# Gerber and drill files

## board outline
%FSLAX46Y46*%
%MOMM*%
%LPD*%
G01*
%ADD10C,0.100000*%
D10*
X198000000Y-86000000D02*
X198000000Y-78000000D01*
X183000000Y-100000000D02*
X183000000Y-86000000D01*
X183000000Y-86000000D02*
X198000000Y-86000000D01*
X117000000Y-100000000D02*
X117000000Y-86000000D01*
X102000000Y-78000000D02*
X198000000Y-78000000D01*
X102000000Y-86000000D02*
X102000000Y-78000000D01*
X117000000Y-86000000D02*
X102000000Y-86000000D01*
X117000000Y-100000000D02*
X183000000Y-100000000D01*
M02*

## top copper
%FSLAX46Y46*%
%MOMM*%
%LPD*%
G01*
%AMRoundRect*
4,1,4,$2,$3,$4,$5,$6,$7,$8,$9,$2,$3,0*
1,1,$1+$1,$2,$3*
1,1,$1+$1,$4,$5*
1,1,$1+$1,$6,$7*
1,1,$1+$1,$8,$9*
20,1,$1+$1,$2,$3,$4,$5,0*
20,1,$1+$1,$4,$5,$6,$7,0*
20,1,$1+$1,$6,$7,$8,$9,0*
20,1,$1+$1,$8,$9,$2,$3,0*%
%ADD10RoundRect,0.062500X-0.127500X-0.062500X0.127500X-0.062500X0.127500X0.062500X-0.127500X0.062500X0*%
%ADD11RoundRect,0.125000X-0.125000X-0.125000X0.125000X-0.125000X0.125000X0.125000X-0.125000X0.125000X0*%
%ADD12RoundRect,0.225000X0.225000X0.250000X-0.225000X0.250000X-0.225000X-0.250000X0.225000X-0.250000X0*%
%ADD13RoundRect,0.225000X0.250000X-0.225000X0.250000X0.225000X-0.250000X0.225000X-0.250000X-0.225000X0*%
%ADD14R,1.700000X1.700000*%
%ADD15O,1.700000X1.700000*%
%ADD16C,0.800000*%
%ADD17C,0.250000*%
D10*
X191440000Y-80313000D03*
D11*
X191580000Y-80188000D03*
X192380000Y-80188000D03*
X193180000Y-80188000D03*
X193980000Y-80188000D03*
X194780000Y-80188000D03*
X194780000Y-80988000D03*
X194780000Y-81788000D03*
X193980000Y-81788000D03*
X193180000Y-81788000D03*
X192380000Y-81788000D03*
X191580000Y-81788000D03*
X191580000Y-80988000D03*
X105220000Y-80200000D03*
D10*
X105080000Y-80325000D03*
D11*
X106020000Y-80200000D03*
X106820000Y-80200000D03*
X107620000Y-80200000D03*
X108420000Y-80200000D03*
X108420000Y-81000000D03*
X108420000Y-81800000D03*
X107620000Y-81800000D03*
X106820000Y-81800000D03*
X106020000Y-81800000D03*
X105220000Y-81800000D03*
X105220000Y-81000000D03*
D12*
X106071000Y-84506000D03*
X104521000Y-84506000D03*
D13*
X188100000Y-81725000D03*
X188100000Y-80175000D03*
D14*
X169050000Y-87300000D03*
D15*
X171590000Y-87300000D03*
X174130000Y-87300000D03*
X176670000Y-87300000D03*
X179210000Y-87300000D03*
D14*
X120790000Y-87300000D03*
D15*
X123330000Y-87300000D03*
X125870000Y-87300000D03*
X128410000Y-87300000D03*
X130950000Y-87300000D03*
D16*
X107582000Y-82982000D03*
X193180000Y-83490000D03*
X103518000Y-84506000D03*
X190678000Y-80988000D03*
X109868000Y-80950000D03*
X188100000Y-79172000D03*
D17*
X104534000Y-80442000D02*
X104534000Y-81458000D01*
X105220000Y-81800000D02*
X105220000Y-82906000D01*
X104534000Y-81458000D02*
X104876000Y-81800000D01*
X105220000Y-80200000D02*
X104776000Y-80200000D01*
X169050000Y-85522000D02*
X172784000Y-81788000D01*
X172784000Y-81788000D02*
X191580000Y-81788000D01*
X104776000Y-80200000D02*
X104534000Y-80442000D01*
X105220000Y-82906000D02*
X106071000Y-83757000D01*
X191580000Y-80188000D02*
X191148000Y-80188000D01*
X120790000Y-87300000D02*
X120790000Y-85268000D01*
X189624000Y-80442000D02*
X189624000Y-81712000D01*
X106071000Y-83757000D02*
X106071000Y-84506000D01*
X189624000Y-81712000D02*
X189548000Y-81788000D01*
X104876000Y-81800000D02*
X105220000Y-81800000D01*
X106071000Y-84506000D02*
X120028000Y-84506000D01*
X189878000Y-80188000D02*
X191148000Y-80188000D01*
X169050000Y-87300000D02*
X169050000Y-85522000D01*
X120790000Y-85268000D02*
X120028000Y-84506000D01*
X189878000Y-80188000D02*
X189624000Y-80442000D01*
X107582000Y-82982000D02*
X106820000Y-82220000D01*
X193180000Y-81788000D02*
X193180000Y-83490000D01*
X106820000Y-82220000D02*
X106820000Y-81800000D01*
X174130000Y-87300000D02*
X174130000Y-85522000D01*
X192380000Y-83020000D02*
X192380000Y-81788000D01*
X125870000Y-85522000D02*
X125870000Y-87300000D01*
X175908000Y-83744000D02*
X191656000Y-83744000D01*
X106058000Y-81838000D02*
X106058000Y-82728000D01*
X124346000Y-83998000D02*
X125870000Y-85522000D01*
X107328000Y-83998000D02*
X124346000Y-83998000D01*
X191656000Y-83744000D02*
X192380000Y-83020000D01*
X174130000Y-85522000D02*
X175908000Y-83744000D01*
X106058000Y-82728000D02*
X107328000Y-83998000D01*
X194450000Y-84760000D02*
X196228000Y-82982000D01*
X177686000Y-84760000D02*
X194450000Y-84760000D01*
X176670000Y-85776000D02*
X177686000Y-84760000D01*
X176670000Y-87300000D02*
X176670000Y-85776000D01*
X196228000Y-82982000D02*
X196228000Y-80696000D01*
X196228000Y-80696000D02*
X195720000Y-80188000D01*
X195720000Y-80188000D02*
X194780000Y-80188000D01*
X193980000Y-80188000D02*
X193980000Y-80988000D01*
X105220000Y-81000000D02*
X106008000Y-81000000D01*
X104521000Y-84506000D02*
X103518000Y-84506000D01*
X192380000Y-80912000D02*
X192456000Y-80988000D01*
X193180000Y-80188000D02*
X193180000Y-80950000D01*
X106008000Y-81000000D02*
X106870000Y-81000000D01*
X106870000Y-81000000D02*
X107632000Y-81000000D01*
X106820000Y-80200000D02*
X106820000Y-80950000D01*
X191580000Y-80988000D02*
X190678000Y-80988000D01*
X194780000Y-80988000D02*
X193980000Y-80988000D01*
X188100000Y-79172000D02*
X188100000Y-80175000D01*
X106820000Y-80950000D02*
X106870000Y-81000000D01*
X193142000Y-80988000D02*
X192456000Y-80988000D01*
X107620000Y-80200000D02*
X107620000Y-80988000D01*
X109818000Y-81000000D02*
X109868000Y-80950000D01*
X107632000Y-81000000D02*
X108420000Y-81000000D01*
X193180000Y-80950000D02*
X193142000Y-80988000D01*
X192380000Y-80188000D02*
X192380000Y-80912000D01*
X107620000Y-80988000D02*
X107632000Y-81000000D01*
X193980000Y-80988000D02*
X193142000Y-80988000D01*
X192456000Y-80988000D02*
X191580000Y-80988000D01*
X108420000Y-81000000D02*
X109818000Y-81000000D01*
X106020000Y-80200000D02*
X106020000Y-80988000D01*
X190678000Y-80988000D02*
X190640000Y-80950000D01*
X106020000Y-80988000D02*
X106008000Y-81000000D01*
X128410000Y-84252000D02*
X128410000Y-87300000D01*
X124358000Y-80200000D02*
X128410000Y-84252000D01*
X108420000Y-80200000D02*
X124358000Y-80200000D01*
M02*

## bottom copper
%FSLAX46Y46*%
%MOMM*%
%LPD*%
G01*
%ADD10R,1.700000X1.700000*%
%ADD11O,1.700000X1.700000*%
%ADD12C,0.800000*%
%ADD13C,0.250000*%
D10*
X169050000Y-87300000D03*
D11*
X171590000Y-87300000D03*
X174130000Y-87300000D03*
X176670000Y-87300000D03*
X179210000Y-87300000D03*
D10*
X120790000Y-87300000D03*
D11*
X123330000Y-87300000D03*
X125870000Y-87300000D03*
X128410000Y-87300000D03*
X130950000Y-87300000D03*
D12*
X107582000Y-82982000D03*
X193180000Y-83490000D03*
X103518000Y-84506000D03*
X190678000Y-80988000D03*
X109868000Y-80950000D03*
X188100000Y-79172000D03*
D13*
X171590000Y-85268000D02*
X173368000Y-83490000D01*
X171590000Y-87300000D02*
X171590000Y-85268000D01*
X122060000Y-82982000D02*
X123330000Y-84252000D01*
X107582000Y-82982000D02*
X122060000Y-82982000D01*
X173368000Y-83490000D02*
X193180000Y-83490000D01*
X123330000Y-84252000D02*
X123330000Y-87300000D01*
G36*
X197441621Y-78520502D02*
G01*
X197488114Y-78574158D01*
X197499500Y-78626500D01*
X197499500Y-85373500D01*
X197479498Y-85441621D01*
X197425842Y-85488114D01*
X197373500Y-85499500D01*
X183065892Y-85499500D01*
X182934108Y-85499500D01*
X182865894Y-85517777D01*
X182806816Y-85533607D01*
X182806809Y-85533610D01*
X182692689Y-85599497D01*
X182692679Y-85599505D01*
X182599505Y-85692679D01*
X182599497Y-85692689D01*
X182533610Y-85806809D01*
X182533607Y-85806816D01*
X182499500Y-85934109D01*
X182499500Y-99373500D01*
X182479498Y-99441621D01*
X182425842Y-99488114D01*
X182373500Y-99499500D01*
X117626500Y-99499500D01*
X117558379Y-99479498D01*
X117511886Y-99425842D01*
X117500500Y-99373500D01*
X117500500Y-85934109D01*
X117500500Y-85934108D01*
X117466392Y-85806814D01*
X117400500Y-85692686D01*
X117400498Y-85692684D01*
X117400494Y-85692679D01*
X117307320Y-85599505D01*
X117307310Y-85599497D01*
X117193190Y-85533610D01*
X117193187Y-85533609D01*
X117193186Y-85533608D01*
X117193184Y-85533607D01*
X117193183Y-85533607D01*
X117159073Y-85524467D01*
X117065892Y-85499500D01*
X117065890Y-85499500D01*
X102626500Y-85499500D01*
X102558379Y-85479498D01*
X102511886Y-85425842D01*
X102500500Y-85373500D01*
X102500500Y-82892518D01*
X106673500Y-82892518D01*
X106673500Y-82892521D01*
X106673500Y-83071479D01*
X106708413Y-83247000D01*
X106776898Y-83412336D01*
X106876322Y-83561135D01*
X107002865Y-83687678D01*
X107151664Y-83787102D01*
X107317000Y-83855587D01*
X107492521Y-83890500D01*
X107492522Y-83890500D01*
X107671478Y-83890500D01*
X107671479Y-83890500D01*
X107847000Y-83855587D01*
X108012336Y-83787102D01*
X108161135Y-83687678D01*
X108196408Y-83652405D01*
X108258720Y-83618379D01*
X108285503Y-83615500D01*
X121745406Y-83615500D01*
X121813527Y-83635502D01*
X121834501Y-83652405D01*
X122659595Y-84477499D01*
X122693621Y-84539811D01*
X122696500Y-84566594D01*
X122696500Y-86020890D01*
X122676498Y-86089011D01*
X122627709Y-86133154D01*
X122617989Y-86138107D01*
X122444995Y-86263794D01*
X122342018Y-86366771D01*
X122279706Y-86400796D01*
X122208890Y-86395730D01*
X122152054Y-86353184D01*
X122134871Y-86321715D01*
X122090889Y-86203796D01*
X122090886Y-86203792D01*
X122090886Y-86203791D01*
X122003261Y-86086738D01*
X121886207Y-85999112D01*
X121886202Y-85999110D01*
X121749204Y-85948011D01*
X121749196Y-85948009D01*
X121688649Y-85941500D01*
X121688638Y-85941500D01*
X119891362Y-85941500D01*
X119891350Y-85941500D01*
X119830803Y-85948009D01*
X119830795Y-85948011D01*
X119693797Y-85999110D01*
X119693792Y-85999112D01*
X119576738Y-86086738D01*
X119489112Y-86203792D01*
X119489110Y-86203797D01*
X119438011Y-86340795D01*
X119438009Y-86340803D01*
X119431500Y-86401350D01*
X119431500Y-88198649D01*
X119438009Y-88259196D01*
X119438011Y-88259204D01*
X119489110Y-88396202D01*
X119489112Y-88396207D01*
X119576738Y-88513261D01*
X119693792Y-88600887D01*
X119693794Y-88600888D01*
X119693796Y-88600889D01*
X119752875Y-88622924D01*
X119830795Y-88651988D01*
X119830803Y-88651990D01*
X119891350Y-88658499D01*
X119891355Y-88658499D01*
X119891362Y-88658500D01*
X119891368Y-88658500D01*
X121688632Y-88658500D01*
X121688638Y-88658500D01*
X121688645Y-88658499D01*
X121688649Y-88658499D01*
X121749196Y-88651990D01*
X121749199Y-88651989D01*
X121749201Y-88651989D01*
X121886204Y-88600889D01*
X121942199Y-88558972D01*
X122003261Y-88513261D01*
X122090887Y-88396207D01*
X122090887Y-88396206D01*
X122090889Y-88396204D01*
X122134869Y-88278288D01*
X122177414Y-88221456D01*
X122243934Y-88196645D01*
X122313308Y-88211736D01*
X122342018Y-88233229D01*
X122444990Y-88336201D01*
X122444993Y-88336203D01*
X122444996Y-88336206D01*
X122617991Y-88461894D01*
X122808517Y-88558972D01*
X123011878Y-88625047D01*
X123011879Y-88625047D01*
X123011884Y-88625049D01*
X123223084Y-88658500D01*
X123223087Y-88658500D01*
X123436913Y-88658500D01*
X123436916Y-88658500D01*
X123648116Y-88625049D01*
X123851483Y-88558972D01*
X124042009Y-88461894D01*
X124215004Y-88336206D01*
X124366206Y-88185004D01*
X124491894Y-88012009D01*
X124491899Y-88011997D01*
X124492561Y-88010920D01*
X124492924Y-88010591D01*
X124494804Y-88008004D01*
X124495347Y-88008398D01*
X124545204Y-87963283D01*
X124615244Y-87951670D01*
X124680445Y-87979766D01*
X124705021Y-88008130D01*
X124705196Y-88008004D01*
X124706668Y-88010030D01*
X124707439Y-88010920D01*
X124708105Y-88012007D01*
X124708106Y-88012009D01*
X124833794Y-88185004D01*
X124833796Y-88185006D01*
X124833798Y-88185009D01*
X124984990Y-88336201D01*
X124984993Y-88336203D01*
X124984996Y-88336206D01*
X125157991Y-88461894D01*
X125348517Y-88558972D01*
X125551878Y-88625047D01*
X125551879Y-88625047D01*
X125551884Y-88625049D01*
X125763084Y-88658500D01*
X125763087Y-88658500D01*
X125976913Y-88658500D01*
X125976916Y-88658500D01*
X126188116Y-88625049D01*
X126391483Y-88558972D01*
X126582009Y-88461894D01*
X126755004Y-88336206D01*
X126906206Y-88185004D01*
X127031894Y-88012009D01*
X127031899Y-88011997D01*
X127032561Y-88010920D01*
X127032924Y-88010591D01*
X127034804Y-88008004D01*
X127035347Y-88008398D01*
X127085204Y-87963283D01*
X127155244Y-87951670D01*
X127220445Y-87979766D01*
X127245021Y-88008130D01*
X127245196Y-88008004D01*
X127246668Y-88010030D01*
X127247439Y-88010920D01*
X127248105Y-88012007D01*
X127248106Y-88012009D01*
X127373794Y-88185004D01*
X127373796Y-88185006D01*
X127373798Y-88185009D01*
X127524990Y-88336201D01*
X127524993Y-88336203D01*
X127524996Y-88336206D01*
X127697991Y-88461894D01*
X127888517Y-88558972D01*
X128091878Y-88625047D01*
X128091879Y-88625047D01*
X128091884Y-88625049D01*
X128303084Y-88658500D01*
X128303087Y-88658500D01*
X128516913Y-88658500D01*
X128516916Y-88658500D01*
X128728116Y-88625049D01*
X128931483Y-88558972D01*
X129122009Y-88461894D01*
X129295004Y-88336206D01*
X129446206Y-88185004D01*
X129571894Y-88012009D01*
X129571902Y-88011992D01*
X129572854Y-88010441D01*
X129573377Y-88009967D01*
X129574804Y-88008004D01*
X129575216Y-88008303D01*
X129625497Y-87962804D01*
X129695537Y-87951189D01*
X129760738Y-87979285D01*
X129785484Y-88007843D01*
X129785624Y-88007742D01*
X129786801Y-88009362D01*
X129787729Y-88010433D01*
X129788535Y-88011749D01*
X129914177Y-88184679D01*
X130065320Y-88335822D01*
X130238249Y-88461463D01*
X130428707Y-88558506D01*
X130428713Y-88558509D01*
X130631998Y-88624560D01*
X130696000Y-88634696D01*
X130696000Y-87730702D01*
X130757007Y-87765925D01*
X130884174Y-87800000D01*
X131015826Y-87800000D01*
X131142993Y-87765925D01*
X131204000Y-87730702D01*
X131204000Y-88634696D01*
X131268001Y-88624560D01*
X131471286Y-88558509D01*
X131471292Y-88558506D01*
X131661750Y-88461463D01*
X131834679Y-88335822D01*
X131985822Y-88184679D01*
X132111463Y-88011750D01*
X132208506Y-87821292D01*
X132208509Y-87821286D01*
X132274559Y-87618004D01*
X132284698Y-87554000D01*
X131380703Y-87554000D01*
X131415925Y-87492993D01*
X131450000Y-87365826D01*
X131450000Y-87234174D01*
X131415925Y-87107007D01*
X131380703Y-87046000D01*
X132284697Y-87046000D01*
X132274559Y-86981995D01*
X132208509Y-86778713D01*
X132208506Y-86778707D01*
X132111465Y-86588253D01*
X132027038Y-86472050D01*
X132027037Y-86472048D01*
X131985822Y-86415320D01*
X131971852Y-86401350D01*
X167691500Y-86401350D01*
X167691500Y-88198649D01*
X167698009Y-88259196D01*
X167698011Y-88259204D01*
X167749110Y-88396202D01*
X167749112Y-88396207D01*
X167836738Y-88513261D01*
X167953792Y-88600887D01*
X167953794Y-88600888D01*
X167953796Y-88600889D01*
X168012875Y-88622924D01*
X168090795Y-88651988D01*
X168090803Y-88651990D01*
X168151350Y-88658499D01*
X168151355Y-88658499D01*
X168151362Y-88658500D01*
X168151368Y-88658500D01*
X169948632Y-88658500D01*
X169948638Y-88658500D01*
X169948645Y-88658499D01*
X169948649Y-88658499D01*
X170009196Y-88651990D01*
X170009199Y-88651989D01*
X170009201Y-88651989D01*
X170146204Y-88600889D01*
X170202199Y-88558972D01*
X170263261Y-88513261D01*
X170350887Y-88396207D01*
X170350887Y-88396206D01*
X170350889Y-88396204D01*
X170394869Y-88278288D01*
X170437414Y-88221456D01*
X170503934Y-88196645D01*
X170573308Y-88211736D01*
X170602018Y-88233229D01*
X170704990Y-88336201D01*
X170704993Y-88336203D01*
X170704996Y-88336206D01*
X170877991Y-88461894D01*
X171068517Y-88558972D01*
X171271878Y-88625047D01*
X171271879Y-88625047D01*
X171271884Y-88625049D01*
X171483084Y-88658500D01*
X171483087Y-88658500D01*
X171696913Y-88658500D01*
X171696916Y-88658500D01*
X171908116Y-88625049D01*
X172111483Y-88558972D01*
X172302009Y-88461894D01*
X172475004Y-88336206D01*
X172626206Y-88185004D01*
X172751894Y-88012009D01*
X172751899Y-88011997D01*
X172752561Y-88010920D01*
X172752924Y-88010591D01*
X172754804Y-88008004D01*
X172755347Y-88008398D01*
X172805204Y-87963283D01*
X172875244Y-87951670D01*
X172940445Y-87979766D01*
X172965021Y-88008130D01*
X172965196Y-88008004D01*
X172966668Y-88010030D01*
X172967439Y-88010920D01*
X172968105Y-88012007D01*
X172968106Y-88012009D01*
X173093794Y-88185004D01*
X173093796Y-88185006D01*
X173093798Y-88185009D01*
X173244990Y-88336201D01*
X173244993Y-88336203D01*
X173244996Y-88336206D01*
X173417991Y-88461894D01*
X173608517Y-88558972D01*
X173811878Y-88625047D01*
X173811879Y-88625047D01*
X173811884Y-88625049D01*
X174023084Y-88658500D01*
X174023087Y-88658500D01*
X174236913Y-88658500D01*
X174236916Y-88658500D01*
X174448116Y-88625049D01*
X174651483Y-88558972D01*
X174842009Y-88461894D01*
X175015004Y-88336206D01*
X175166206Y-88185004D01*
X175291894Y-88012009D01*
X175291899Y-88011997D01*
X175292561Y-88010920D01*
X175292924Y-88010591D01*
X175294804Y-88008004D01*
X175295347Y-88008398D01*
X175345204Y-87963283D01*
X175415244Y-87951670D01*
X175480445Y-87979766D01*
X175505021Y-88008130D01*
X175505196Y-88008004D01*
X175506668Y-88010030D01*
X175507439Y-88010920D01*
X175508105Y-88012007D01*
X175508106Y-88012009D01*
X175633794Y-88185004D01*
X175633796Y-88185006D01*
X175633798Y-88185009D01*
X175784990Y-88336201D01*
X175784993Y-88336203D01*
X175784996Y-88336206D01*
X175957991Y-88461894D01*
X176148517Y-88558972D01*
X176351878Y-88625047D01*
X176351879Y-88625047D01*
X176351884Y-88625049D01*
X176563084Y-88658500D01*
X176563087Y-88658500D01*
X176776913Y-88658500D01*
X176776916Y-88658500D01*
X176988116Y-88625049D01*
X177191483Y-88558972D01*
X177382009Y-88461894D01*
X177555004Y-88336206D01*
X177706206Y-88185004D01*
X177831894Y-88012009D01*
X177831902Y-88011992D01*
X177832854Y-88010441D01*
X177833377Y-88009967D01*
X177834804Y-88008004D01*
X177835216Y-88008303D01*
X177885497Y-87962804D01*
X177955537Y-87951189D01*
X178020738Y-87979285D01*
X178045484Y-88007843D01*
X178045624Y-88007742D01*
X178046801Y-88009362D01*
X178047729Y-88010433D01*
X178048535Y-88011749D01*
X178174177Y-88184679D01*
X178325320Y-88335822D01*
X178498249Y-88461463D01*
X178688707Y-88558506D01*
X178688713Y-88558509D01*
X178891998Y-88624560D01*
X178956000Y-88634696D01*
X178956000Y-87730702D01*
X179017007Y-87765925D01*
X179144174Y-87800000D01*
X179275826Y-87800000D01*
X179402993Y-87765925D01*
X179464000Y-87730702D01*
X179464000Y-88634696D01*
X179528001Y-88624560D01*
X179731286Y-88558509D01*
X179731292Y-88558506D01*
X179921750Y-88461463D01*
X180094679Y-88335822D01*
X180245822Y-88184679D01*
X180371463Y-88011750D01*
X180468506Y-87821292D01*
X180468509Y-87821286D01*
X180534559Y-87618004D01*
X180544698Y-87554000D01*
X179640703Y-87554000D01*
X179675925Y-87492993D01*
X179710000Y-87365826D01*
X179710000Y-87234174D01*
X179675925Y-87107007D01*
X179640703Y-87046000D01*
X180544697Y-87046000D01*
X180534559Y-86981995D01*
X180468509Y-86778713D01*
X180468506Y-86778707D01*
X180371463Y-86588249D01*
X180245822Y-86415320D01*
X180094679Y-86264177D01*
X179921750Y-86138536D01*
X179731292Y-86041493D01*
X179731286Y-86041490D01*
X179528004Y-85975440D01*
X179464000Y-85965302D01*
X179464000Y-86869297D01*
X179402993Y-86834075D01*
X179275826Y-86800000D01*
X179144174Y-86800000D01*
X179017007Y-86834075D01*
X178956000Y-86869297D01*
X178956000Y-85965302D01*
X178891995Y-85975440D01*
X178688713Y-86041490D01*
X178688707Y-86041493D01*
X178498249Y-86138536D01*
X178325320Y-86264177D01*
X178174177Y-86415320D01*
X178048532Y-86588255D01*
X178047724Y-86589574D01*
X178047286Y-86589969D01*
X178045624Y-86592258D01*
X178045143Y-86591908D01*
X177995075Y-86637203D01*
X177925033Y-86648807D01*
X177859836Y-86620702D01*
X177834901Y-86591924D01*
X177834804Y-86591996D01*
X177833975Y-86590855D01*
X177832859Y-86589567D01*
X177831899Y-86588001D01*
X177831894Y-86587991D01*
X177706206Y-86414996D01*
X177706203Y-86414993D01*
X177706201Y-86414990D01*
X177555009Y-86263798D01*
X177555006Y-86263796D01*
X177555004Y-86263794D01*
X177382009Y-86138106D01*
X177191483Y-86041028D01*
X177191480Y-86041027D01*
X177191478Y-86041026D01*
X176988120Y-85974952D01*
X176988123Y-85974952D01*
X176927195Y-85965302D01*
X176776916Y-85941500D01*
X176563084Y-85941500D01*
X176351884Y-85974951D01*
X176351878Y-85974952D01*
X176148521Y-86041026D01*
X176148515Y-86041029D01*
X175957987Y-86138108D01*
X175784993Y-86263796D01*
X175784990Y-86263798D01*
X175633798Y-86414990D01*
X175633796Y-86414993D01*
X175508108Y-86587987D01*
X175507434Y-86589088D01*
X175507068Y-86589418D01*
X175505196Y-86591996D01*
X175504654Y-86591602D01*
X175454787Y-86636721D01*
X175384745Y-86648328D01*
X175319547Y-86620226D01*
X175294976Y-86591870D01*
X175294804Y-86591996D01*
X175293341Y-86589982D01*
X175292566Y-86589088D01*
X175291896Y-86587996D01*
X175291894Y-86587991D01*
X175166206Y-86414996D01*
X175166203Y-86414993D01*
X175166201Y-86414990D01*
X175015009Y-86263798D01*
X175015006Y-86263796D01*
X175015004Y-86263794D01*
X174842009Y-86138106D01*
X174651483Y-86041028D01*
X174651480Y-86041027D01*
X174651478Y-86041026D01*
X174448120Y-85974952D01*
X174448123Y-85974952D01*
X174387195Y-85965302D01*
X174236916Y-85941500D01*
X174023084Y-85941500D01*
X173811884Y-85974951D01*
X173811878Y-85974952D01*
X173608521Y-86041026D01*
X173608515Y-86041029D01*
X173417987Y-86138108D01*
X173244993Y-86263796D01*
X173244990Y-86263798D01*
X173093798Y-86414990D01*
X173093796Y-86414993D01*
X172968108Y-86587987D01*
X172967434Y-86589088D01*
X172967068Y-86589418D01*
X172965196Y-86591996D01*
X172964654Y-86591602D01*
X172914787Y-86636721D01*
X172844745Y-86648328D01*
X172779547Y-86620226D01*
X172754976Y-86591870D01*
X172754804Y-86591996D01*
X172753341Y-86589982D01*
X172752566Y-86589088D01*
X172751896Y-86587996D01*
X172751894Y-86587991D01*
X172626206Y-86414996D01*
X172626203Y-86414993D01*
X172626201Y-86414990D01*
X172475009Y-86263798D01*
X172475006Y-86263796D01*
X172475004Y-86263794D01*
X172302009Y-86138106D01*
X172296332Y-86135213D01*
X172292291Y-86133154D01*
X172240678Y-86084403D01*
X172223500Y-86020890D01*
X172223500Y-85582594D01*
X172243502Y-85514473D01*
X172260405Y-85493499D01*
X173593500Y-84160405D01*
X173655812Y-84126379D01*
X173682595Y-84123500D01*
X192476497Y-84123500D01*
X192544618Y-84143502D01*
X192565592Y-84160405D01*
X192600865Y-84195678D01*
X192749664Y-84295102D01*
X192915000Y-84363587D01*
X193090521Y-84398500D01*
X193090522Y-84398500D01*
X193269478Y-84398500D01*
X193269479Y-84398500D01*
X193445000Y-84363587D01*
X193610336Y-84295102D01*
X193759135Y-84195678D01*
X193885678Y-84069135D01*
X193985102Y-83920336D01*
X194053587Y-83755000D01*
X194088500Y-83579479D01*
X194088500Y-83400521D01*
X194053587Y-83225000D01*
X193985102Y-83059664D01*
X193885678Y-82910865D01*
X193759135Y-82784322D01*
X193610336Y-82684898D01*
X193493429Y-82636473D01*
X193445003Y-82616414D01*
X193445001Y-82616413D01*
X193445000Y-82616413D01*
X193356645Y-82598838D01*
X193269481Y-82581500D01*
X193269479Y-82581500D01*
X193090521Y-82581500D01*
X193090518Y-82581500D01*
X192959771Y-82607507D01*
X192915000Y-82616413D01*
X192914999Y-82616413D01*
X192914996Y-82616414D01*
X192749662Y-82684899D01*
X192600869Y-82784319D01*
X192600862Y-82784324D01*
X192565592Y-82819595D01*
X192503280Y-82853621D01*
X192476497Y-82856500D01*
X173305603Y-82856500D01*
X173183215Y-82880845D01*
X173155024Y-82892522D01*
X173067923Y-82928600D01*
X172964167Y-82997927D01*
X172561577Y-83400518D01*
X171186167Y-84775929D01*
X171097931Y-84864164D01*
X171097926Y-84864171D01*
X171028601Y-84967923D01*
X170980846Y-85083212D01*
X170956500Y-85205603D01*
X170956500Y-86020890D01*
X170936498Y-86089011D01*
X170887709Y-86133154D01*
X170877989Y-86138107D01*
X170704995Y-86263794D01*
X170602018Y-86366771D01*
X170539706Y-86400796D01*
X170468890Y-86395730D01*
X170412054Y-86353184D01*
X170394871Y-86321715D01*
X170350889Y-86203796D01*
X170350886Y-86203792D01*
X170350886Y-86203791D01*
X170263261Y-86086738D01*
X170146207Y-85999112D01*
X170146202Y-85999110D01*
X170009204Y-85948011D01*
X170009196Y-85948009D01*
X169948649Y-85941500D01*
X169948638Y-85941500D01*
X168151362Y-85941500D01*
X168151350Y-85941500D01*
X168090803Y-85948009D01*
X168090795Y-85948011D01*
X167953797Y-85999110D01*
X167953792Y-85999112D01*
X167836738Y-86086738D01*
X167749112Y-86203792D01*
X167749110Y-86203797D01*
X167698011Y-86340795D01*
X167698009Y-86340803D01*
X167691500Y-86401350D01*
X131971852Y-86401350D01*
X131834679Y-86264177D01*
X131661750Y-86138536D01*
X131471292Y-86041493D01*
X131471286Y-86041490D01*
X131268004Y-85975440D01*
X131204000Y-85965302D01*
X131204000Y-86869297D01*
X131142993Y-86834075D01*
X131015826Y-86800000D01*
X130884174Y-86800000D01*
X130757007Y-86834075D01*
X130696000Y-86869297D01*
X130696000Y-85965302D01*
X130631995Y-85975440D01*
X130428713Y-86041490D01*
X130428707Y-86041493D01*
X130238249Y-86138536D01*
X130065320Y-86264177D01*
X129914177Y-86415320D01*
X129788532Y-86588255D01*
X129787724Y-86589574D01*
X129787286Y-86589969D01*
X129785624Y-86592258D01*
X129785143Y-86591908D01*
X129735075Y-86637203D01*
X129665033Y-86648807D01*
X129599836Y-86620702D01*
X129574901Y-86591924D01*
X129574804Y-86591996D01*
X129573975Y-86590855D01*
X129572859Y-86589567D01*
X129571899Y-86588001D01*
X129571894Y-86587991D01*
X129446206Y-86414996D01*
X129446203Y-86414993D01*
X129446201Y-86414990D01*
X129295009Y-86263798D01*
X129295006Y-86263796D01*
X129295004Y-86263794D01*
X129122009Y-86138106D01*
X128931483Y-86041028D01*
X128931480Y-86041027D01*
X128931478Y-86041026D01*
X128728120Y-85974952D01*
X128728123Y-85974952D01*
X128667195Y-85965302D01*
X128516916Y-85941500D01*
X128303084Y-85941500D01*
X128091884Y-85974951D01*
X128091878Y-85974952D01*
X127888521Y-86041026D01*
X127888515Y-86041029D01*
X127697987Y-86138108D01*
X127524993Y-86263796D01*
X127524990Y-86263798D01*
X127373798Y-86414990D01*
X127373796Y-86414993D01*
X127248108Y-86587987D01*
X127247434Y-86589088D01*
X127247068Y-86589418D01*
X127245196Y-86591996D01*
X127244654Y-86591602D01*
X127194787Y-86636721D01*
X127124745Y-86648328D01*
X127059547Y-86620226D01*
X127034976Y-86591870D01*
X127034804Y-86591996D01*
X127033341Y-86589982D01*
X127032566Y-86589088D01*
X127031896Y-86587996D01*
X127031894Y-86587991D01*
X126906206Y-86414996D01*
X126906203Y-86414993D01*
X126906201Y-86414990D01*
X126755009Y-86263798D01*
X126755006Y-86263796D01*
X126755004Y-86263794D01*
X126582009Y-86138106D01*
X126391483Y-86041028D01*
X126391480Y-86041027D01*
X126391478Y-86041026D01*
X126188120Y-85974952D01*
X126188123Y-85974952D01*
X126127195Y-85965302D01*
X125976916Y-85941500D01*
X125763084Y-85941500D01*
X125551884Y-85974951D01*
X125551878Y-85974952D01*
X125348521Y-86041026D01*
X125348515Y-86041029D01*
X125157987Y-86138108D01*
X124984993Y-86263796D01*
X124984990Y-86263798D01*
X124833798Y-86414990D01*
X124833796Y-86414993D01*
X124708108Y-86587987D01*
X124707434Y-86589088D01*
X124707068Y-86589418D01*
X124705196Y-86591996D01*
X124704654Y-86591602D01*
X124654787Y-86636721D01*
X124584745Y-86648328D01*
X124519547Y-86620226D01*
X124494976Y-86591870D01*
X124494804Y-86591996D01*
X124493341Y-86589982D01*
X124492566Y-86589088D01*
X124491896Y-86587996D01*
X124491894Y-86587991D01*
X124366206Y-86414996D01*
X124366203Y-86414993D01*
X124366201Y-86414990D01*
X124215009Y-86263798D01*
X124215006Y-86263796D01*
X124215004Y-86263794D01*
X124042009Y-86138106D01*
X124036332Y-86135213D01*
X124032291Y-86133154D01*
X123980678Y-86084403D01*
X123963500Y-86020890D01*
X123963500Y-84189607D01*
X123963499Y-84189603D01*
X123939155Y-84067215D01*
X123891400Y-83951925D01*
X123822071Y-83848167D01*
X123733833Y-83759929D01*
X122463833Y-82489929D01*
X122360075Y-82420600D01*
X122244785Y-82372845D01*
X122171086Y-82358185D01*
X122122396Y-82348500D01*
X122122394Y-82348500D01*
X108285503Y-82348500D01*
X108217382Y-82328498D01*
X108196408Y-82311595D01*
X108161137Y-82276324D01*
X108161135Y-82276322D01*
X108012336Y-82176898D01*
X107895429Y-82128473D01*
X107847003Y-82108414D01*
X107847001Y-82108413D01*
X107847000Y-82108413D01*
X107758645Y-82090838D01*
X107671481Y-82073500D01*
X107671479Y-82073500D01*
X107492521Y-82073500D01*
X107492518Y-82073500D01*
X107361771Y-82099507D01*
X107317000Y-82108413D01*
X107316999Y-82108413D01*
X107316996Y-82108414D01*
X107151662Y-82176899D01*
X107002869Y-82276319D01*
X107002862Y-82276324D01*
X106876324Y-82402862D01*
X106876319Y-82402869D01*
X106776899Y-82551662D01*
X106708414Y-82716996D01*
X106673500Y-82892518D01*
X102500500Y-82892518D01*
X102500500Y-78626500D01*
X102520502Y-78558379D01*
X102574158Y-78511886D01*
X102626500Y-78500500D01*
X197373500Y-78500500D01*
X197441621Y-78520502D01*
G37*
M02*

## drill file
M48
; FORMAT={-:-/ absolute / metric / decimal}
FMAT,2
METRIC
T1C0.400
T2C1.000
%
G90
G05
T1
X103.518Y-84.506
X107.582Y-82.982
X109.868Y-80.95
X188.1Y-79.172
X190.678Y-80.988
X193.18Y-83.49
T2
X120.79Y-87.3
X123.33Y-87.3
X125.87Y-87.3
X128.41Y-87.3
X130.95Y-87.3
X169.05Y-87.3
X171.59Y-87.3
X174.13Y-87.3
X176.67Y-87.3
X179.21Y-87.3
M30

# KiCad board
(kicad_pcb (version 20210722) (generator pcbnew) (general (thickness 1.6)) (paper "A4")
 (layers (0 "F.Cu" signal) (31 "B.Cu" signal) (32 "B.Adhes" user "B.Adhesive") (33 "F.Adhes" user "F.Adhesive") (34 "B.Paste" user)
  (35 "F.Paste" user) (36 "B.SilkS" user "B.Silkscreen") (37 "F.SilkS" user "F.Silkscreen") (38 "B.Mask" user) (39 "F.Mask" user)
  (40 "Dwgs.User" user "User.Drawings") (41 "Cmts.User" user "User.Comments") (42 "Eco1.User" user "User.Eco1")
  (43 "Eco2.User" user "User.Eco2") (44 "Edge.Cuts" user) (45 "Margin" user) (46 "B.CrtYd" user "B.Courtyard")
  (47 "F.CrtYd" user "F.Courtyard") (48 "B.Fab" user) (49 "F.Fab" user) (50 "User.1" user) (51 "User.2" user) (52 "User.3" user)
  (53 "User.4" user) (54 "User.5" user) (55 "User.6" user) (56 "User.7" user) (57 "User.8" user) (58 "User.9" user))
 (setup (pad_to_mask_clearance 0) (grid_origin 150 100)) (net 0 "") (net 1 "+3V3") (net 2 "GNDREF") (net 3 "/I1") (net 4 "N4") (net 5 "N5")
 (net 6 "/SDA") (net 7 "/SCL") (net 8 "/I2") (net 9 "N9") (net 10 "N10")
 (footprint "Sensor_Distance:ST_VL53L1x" (layer "F.Cu") (at 193.18 80.988)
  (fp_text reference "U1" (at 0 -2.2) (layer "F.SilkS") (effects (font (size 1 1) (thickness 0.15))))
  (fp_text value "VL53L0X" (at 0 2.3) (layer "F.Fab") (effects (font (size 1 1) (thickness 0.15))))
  (pad "1" smd roundrect locked (at -1.74 -0.675) (size 0.38 0.25) (layers "F.Cu" "F.Paste" "F.Mask") (roundrect_rratio 0.25) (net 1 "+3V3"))
  (pad "1" smd roundrect locked (at -1.6 -0.8) (size 0.5 0.5) (layers "F.Cu" "F.Paste" "F.Mask") (roundrect_rratio 0.25) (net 1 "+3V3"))
  (pad "2" smd roundrect locked (at -0.8 -0.8) (size 0.5 0.5) (layers "F.Cu" "F.Paste" "F.Mask") (roundrect_rratio 0.25) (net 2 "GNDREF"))
  (pad "3" smd roundrect locked (at 0 -0.8) (size 0.5 0.5) (layers "F.Cu" "F.Paste" "F.Mask") (roundrect_rratio 0.25) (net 2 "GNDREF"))
  (pad "4" smd roundrect locked (at 0.8 -0.8) (size 0.5 0.5) (layers "F.Cu" "F.Paste" "F.Mask") (roundrect_rratio 0.25) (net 2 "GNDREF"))
  (pad "5" smd roundrect locked (at 1.6 -0.8) (size 0.5 0.5) (layers "F.Cu" "F.Paste" "F.Mask") (roundrect_rratio 0.25) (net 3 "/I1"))
  (pad "6" smd roundrect locked (at 1.6 0) (size 0.5 0.5) (layers "F.Cu" "F.Paste" "F.Mask") (roundrect_rratio 0.25) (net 2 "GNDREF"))
  (pad "7" smd roundrect locked (at 1.6 0.8) (size 0.5 0.5) (layers "F.Cu" "F.Paste" "F.Mask") (roundrect_rratio 0.25) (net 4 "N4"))
  (pad "8" smd roundrect locked (at 0.8 0.8) (size 0.5 0.5) (layers "F.Cu" "F.Paste" "F.Mask") (roundrect_rratio 0.25) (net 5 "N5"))
  (pad "9" smd roundrect locked (at 0 0.8) (size 0.5 0.5) (layers "F.Cu" "F.Paste" "F.Mask") (roundrect_rratio 0.25) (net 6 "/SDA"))
  (pad "10" smd roundrect locked (at -0.8 0.8) (size 0.5 0.5) (layers "F.Cu" "F.Paste" "F.Mask") (roundrect_rratio 0.25) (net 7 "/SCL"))
  (pad "11" smd roundrect locked (at -1.6 0.8) (size 0.5 0.5) (layers "F.Cu" "F.Paste" "F.Mask") (roundrect_rratio 0.25) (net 1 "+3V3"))
  (pad "12" smd roundrect locked (at -1.6 0) (size 0.5 0.5) (layers "F.Cu" "F.Paste" "F.Mask") (roundrect_rratio 0.25) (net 2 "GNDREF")))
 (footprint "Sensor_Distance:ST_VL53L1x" (layer "F.Cu") (at 106.82 81)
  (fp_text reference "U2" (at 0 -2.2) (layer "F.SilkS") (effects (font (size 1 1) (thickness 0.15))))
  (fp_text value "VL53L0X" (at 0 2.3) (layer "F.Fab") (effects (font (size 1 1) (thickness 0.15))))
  (pad "1" smd roundrect locked (at -1.6 -0.8) (size 0.5 0.5) (layers "F.Cu" "F.Paste" "F.Mask") (roundrect_rratio 0.25) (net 1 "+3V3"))
  (pad "1" smd roundrect locked (at -1.74 -0.675) (size 0.38 0.25) (layers "F.Cu" "F.Paste" "F.Mask") (roundrect_rratio 0.25) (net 1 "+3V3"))
  (pad "2" smd roundrect locked (at -0.8 -0.8) (size 0.5 0.5) (layers "F.Cu" "F.Paste" "F.Mask") (roundrect_rratio 0.25) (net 2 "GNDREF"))
  (pad "3" smd roundrect locked (at 0 -0.8) (size 0.5 0.5) (layers "F.Cu" "F.Paste" "F.Mask") (roundrect_rratio 0.25) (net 2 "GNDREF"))
  (pad "4" smd roundrect locked (at 0.8 -0.8) (size 0.5 0.5) (layers "F.Cu" "F.Paste" "F.Mask") (roundrect_rratio 0.25) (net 2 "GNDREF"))
  (pad "5" smd roundrect locked (at 1.6 -0.8) (size 0.5 0.5) (layers "F.Cu" "F.Paste" "F.Mask") (roundrect_rratio 0.25) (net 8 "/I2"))
  (pad "6" smd roundrect locked (at 1.6 0) (size 0.5 0.5) (layers "F.Cu" "F.Paste" "F.Mask") (roundrect_rratio 0.25) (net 2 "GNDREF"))
  (pad "7" smd roundrect locked (at 1.6 0.8) (size 0.5 0.5) (layers "F.Cu" "F.Paste" "F.Mask") (roundrect_rratio 0.25) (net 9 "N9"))
  (pad "8" smd roundrect locked (at 0.8 0.8) (size 0.5 0.5) (layers "F.Cu" "F.Paste" "F.Mask") (roundrect_rratio 0.25) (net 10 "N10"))
  (pad "9" smd roundrect locked (at 0 0.8) (size 0.5 0.5) (layers "F.Cu" "F.Paste" "F.Mask") (roundrect_rratio 0.25) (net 6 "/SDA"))
  (pad "10" smd roundrect locked (at -0.8 0.8) (size 0.5 0.5) (layers "F.Cu" "F.Paste" "F.Mask") (roundrect_rratio 0.25) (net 7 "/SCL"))
  (pad "11" smd roundrect locked (at -1.6 0.8) (size 0.5 0.5) (layers "F.Cu" "F.Paste" "F.Mask") (roundrect_rratio 0.25) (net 1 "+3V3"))
  (pad "12" smd roundrect locked (at -1.6 0) (size 0.5 0.5) (layers "F.Cu" "F.Paste" "F.Mask") (roundrect_rratio 0.25) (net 2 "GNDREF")))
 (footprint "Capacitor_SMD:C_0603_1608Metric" (layer "F.Cu") (at 105.296 84.506 180)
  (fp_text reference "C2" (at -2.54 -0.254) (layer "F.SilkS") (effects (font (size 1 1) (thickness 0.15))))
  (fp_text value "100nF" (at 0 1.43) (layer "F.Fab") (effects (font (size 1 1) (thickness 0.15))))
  (pad "1" smd roundrect locked (at -0.775 0 180) (size 0.9 0.95) (layers "F.Cu" "F.Paste" "F.Mask") (roundrect_rratio 0.25) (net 1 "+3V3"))
  (pad "2" smd roundrect locked (at 0.775 0 180) (size 0.9 0.95) (layers "F.Cu" "F.Paste" "F.Mask") (roundrect_rratio 0.25) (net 2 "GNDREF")))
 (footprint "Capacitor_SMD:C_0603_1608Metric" (layer "F.Cu") (at 188.1 80.95 90)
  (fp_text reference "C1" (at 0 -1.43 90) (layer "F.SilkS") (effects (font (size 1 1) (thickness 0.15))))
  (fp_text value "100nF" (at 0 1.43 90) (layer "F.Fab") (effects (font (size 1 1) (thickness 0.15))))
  (pad "1" smd roundrect locked (at -0.775 0 90) (size 0.9 0.95) (layers "F.Cu" "F.Paste" "F.Mask") (roundrect_rratio 0.25) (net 1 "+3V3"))
  (pad "2" smd roundrect locked (at 0.775 0 90) (size 0.9 0.95) (layers "F.Cu" "F.Paste" "F.Mask") (roundrect_rratio 0.25) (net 2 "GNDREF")))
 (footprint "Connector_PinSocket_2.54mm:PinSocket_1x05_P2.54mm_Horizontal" (layer "F.Cu") (at 169.05 87.3 90)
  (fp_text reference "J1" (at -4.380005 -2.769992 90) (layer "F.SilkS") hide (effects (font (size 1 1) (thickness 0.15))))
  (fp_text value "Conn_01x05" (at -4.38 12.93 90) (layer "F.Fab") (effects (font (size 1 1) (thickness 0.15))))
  (pad "1" thru_hole rect locked (at 0 0 90) (size 1.7 1.7) (drill 1) (layers *.Cu *.Mask) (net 1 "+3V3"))
  (pad "2" thru_hole oval locked (at 0 2.54 90) (size 1.7 1.7) (drill 1) (layers *.Cu *.Mask) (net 6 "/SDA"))
  (pad "3" thru_hole oval locked (at 0 5.08 90) (size 1.7 1.7) (drill 1) (layers *.Cu *.Mask) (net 7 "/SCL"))
  (pad "4" thru_hole oval locked (at 0 7.62 90) (size 1.7 1.7) (drill 1) (layers *.Cu *.Mask) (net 3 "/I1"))
  (pad "5" thru_hole oval locked (at 0 10.16 90) (size 1.7 1.7) (drill 1) (layers *.Cu *.Mask) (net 2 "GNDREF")))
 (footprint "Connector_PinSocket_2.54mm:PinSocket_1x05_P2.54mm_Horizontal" (layer "F.Cu") (at 120.79 87.3 90)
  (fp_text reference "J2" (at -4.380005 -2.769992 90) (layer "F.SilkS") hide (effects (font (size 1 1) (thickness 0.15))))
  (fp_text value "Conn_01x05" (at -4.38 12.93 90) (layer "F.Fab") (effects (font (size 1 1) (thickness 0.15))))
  (pad "1" thru_hole rect locked (at 0 0 90) (size 1.7 1.7) (drill 1) (layers *.Cu *.Mask) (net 1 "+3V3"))
  (pad "2" thru_hole oval locked (at 0 2.54 90) (size 1.7 1.7) (drill 1) (layers *.Cu *.Mask) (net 6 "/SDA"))
  (pad "3" thru_hole oval locked (at 0 5.08 90) (size 1.7 1.7) (drill 1) (layers *.Cu *.Mask) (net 7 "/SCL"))
  (pad "4" thru_hole oval locked (at 0 7.62 90) (size 1.7 1.7) (drill 1) (layers *.Cu *.Mask) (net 8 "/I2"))
  (pad "5" thru_hole oval locked (at 0 10.16 90) (size 1.7 1.7) (drill 1) (layers *.Cu *.Mask) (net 2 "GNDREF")))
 (gr_line (start 198 86) (end 198 78) (layer "Edge.Cuts") (width 0.1))
 (gr_line (start 183 100) (end 183 86) (layer "Edge.Cuts") (width 0.1))
 (gr_line (start 183 86) (end 198 86) (layer "Edge.Cuts") (width 0.1))
 (gr_line (start 117 100) (end 117 86) (layer "Edge.Cuts") (width 0.1))
 (gr_line (start 102 78) (end 198 78) (layer "Edge.Cuts") (width 0.1))
 (gr_line (start 102 86) (end 102 78) (layer "Edge.Cuts") (width 0.1))
 (gr_line (start 117 86) (end 102 86) (layer "Edge.Cuts") (width 0.1))
 (gr_line (start 117 100) (end 183 100) (layer "Edge.Cuts") (width 0.1))
 (segment (start 104.534 80.442) (end 104.534 81.458) (width 0.25) (layer "F.Cu") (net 1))
 (segment (start 105.22 81.8) (end 105.22 82.906) (width 0.25) (layer "F.Cu") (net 1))
 (segment (start 104.534 81.458) (end 104.876 81.8) (width 0.25) (layer "F.Cu") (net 1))
 (segment (start 105.22 80.2) (end 104.776 80.2) (width 0.25) (layer "F.Cu") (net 1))
 (segment (start 169.05 85.522) (end 172.784 81.788) (width 0.25) (layer "F.Cu") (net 1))
 (segment (start 172.784 81.788) (end 191.58 81.788) (width 0.25) (layer "F.Cu") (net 1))
 (segment (start 104.776 80.2) (end 104.534 80.442) (width 0.25) (layer "F.Cu") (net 1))
 (segment (start 105.22 82.906) (end 106.071 83.757) (width 0.25) (layer "F.Cu") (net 1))
 (segment (start 191.58 80.188) (end 191.148 80.188) (width 0.25) (layer "F.Cu") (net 1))
 (segment (start 120.79 87.3) (end 120.79 85.268) (width 0.25) (layer "F.Cu") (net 1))
 (segment (start 189.624 80.442) (end 189.624 81.712) (width 0.25) (layer "F.Cu") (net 1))
 (segment (start 106.071 83.757) (end 106.071 84.506) (width 0.25) (layer "F.Cu") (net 1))
 (segment (start 189.624 81.712) (end 189.548 81.788) (width 0.25) (layer "F.Cu") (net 1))
 (segment (start 104.876 81.8) (end 105.22 81.8) (width 0.25) (layer "F.Cu") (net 1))
 (segment (start 106.071 84.506) (end 120.028 84.506) (width 0.25) (layer "F.Cu") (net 1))
 (segment (start 189.878 80.188) (end 191.148 80.188) (width 0.25) (layer "F.Cu") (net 1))
 (segment (start 169.05 87.3) (end 169.05 85.522) (width 0.25) (layer "F.Cu") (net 1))
 (segment (start 120.79 85.268) (end 120.028 84.506) (width 0.25) (layer "F.Cu") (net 1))
 (segment (start 189.878 80.188) (end 189.624 80.442) (width 0.25) (layer "F.Cu") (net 1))
 (segment (start 107.582 82.982) (end 106.82 82.22) (width 0.25) (layer "F.Cu") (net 6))
 (segment (start 193.18 81.788) (end 193.18 83.49) (width 0.25) (layer "F.Cu") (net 6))
 (segment (start 106.82 82.22) (end 106.82 81.8) (width 0.25) (layer "F.Cu") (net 6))
 (via (at 107.582 82.982) (size 0.8) (drill 0.4) (layers "F.Cu" "B.Cu") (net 6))
 (via (at 193.18 83.49) (size 0.8) (drill 0.4) (layers "F.Cu" "B.Cu") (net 6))
 (segment (start 171.59 85.268) (end 173.368 83.49) (width 0.25) (layer "B.Cu") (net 6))
 (segment (start 171.59 87.3) (end 171.59 85.268) (width 0.25) (layer "B.Cu") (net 6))
 (segment (start 122.06 82.982) (end 123.33 84.252) (width 0.25) (layer "B.Cu") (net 6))
 (segment (start 107.582 82.982) (end 122.06 82.982) (width 0.25) (layer "B.Cu") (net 6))
 (segment (start 173.368 83.49) (end 193.18 83.49) (width 0.25) (layer "B.Cu") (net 6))
 (segment (start 123.33 84.252) (end 123.33 87.3) (width 0.25) (layer "B.Cu") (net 6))
 (segment (start 174.13 87.3) (end 174.13 85.522) (width 0.25) (layer "F.Cu") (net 7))
 (segment (start 192.38 83.02) (end 192.38 81.788) (width 0.25) (layer "F.Cu") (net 7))
 (segment (start 125.87 85.522) (end 125.87 87.3) (width 0.25) (layer "F.Cu") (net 7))
 (segment (start 175.908 83.744) (end 191.656 83.744) (width 0.25) (layer "F.Cu") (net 7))
 (segment (start 106.058 81.838) (end 106.058 82.728) (width 0.25) (layer "F.Cu") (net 7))
 (segment (start 124.346 83.998) (end 125.87 85.522) (width 0.25) (layer "F.Cu") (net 7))
 (segment (start 107.328 83.998) (end 124.346 83.998) (width 0.25) (layer "F.Cu") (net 7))
 (segment (start 191.656 83.744) (end 192.38 83.02) (width 0.25) (layer "F.Cu") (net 7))
 (segment (start 174.13 85.522) (end 175.908 83.744) (width 0.25) (layer "F.Cu") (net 7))
 (segment (start 106.058 82.728) (end 107.328 83.998) (width 0.25) (layer "F.Cu") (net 7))
 (segment (start 194.45 84.76) (end 196.228 82.982) (width 0.25) (layer "F.Cu") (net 3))
 (segment (start 177.686 84.76) (end 194.45 84.76) (width 0.25) (layer "F.Cu") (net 3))
 (segment (start 176.67 85.776) (end 177.686 84.76) (width 0.25) (layer "F.Cu") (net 3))
 (segment (start 176.67 87.3) (end 176.67 85.776) (width 0.25) (layer "F.Cu") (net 3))
 (segment (start 196.228 82.982) (end 196.228 80.696) (width 0.25) (layer "F.Cu") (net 3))
 (segment (start 196.228 80.696) (end 195.72 80.188) (width 0.25) (layer "F.Cu") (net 3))
 (segment (start 195.72 80.188) (end 194.78 80.188) (width 0.25) (layer "F.Cu") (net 3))
 (segment (start 193.98 80.188) (end 193.98 80.988) (width 0.25) (layer "F.Cu") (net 2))
 (segment (start 105.22 81) (end 106.008 81) (width 0.25) (layer "F.Cu") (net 2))
 (segment (start 104.521 84.506) (end 103.518 84.506) (width 0.25) (layer "F.Cu") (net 2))
 (segment (start 192.38 80.912) (end 192.456 80.988) (width 0.25) (layer "F.Cu") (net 2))
 (segment (start 193.18 80.188) (end 193.18 80.95) (width 0.25) (layer "F.Cu") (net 2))
 (segment (start 106.008 81) (end 106.87 81) (width 0.25) (layer "F.Cu") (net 2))
 (segment (start 106.87 81) (end 107.632 81) (width 0.25) (layer "F.Cu") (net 2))
 (segment (start 106.82 80.2) (end 106.82 80.95) (width 0.25) (layer "F.Cu") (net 2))
 (segment (start 191.58 80.988) (end 190.678 80.988) (width 0.25) (layer "F.Cu") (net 2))
 (segment (start 194.78 80.988) (end 193.98 80.988) (width 0.25) (layer "F.Cu") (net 2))
 (segment (start 188.1 79.172) (end 188.1 80.175) (width 0.25) (layer "F.Cu") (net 2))
 (segment (start 106.82 80.95) (end 106.87 81) (width 0.25) (layer "F.Cu") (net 2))
 (segment (start 193.142 80.988) (end 192.456 80.988) (width 0.25) (layer "F.Cu") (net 2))
 (segment (start 107.62 80.2) (end 107.62 80.988) (width 0.25) (layer "F.Cu") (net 2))
 (segment (start 109.818 81) (end 109.868 80.95) (width 0.25) (layer "F.Cu") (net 2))
 (segment (start 107.632 81) (end 108.42 81) (width 0.25) (layer "F.Cu") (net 2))
 (segment (start 193.18 80.95) (end 193.142 80.988) (width 0.25) (layer "F.Cu") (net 2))
 (segment (start 192.38 80.188) (end 192.38 80.912) (width 0.25) (layer "F.Cu") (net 2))
 (segment (start 107.62 80.988) (end 107.632 81) (width 0.25) (layer "F.Cu") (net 2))
 (segment (start 193.98 80.988) (end 193.142 80.988) (width 0.25) (layer "F.Cu") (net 2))
 (segment (start 192.456 80.988) (end 191.58 80.988) (width 0.25) (layer "F.Cu") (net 2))
 (segment (start 108.42 81) (end 109.818 81) (width 0.25) (layer "F.Cu") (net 2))
 (segment (start 106.02 80.2) (end 106.02 80.988) (width 0.25) (layer "F.Cu") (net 2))
 (segment (start 190.678 80.988) (end 190.64 80.95) (width 0.25) (layer "F.Cu") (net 2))
 (segment (start 106.02 80.988) (end 106.008 81) (width 0.25) (layer "F.Cu") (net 2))
 (via (at 103.518 84.506) (size 0.8) (drill 0.4) (layers "F.Cu" "B.Cu") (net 2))
 (via (at 190.678 80.988) (size 0.8) (drill 0.4) (layers "F.Cu" "B.Cu") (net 2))
 (via (at 109.868 80.95) (size 0.8) (drill 0.4) (layers "F.Cu" "B.Cu") (free) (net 2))
 (via (at 188.1 79.172) (size 0.8) (drill 0.4) (layers "F.Cu" "B.Cu") (free) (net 2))
 (segment (start 128.41 84.252) (end 128.41 87.3) (width 0.25) (layer "F.Cu") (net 8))
 (segment (start 124.358 80.2) (end 128.41 84.252) (width 0.25) (layer "F.Cu") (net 8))
 (segment (start 108.42 80.2) (end 124.358 80.2) (width 0.25) (layer "F.Cu") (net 8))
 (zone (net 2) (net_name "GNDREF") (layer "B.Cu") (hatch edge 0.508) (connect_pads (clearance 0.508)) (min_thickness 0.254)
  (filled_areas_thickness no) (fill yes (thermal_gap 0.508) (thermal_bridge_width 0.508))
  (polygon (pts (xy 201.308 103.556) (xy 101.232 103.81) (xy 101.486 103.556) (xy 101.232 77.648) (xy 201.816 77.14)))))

